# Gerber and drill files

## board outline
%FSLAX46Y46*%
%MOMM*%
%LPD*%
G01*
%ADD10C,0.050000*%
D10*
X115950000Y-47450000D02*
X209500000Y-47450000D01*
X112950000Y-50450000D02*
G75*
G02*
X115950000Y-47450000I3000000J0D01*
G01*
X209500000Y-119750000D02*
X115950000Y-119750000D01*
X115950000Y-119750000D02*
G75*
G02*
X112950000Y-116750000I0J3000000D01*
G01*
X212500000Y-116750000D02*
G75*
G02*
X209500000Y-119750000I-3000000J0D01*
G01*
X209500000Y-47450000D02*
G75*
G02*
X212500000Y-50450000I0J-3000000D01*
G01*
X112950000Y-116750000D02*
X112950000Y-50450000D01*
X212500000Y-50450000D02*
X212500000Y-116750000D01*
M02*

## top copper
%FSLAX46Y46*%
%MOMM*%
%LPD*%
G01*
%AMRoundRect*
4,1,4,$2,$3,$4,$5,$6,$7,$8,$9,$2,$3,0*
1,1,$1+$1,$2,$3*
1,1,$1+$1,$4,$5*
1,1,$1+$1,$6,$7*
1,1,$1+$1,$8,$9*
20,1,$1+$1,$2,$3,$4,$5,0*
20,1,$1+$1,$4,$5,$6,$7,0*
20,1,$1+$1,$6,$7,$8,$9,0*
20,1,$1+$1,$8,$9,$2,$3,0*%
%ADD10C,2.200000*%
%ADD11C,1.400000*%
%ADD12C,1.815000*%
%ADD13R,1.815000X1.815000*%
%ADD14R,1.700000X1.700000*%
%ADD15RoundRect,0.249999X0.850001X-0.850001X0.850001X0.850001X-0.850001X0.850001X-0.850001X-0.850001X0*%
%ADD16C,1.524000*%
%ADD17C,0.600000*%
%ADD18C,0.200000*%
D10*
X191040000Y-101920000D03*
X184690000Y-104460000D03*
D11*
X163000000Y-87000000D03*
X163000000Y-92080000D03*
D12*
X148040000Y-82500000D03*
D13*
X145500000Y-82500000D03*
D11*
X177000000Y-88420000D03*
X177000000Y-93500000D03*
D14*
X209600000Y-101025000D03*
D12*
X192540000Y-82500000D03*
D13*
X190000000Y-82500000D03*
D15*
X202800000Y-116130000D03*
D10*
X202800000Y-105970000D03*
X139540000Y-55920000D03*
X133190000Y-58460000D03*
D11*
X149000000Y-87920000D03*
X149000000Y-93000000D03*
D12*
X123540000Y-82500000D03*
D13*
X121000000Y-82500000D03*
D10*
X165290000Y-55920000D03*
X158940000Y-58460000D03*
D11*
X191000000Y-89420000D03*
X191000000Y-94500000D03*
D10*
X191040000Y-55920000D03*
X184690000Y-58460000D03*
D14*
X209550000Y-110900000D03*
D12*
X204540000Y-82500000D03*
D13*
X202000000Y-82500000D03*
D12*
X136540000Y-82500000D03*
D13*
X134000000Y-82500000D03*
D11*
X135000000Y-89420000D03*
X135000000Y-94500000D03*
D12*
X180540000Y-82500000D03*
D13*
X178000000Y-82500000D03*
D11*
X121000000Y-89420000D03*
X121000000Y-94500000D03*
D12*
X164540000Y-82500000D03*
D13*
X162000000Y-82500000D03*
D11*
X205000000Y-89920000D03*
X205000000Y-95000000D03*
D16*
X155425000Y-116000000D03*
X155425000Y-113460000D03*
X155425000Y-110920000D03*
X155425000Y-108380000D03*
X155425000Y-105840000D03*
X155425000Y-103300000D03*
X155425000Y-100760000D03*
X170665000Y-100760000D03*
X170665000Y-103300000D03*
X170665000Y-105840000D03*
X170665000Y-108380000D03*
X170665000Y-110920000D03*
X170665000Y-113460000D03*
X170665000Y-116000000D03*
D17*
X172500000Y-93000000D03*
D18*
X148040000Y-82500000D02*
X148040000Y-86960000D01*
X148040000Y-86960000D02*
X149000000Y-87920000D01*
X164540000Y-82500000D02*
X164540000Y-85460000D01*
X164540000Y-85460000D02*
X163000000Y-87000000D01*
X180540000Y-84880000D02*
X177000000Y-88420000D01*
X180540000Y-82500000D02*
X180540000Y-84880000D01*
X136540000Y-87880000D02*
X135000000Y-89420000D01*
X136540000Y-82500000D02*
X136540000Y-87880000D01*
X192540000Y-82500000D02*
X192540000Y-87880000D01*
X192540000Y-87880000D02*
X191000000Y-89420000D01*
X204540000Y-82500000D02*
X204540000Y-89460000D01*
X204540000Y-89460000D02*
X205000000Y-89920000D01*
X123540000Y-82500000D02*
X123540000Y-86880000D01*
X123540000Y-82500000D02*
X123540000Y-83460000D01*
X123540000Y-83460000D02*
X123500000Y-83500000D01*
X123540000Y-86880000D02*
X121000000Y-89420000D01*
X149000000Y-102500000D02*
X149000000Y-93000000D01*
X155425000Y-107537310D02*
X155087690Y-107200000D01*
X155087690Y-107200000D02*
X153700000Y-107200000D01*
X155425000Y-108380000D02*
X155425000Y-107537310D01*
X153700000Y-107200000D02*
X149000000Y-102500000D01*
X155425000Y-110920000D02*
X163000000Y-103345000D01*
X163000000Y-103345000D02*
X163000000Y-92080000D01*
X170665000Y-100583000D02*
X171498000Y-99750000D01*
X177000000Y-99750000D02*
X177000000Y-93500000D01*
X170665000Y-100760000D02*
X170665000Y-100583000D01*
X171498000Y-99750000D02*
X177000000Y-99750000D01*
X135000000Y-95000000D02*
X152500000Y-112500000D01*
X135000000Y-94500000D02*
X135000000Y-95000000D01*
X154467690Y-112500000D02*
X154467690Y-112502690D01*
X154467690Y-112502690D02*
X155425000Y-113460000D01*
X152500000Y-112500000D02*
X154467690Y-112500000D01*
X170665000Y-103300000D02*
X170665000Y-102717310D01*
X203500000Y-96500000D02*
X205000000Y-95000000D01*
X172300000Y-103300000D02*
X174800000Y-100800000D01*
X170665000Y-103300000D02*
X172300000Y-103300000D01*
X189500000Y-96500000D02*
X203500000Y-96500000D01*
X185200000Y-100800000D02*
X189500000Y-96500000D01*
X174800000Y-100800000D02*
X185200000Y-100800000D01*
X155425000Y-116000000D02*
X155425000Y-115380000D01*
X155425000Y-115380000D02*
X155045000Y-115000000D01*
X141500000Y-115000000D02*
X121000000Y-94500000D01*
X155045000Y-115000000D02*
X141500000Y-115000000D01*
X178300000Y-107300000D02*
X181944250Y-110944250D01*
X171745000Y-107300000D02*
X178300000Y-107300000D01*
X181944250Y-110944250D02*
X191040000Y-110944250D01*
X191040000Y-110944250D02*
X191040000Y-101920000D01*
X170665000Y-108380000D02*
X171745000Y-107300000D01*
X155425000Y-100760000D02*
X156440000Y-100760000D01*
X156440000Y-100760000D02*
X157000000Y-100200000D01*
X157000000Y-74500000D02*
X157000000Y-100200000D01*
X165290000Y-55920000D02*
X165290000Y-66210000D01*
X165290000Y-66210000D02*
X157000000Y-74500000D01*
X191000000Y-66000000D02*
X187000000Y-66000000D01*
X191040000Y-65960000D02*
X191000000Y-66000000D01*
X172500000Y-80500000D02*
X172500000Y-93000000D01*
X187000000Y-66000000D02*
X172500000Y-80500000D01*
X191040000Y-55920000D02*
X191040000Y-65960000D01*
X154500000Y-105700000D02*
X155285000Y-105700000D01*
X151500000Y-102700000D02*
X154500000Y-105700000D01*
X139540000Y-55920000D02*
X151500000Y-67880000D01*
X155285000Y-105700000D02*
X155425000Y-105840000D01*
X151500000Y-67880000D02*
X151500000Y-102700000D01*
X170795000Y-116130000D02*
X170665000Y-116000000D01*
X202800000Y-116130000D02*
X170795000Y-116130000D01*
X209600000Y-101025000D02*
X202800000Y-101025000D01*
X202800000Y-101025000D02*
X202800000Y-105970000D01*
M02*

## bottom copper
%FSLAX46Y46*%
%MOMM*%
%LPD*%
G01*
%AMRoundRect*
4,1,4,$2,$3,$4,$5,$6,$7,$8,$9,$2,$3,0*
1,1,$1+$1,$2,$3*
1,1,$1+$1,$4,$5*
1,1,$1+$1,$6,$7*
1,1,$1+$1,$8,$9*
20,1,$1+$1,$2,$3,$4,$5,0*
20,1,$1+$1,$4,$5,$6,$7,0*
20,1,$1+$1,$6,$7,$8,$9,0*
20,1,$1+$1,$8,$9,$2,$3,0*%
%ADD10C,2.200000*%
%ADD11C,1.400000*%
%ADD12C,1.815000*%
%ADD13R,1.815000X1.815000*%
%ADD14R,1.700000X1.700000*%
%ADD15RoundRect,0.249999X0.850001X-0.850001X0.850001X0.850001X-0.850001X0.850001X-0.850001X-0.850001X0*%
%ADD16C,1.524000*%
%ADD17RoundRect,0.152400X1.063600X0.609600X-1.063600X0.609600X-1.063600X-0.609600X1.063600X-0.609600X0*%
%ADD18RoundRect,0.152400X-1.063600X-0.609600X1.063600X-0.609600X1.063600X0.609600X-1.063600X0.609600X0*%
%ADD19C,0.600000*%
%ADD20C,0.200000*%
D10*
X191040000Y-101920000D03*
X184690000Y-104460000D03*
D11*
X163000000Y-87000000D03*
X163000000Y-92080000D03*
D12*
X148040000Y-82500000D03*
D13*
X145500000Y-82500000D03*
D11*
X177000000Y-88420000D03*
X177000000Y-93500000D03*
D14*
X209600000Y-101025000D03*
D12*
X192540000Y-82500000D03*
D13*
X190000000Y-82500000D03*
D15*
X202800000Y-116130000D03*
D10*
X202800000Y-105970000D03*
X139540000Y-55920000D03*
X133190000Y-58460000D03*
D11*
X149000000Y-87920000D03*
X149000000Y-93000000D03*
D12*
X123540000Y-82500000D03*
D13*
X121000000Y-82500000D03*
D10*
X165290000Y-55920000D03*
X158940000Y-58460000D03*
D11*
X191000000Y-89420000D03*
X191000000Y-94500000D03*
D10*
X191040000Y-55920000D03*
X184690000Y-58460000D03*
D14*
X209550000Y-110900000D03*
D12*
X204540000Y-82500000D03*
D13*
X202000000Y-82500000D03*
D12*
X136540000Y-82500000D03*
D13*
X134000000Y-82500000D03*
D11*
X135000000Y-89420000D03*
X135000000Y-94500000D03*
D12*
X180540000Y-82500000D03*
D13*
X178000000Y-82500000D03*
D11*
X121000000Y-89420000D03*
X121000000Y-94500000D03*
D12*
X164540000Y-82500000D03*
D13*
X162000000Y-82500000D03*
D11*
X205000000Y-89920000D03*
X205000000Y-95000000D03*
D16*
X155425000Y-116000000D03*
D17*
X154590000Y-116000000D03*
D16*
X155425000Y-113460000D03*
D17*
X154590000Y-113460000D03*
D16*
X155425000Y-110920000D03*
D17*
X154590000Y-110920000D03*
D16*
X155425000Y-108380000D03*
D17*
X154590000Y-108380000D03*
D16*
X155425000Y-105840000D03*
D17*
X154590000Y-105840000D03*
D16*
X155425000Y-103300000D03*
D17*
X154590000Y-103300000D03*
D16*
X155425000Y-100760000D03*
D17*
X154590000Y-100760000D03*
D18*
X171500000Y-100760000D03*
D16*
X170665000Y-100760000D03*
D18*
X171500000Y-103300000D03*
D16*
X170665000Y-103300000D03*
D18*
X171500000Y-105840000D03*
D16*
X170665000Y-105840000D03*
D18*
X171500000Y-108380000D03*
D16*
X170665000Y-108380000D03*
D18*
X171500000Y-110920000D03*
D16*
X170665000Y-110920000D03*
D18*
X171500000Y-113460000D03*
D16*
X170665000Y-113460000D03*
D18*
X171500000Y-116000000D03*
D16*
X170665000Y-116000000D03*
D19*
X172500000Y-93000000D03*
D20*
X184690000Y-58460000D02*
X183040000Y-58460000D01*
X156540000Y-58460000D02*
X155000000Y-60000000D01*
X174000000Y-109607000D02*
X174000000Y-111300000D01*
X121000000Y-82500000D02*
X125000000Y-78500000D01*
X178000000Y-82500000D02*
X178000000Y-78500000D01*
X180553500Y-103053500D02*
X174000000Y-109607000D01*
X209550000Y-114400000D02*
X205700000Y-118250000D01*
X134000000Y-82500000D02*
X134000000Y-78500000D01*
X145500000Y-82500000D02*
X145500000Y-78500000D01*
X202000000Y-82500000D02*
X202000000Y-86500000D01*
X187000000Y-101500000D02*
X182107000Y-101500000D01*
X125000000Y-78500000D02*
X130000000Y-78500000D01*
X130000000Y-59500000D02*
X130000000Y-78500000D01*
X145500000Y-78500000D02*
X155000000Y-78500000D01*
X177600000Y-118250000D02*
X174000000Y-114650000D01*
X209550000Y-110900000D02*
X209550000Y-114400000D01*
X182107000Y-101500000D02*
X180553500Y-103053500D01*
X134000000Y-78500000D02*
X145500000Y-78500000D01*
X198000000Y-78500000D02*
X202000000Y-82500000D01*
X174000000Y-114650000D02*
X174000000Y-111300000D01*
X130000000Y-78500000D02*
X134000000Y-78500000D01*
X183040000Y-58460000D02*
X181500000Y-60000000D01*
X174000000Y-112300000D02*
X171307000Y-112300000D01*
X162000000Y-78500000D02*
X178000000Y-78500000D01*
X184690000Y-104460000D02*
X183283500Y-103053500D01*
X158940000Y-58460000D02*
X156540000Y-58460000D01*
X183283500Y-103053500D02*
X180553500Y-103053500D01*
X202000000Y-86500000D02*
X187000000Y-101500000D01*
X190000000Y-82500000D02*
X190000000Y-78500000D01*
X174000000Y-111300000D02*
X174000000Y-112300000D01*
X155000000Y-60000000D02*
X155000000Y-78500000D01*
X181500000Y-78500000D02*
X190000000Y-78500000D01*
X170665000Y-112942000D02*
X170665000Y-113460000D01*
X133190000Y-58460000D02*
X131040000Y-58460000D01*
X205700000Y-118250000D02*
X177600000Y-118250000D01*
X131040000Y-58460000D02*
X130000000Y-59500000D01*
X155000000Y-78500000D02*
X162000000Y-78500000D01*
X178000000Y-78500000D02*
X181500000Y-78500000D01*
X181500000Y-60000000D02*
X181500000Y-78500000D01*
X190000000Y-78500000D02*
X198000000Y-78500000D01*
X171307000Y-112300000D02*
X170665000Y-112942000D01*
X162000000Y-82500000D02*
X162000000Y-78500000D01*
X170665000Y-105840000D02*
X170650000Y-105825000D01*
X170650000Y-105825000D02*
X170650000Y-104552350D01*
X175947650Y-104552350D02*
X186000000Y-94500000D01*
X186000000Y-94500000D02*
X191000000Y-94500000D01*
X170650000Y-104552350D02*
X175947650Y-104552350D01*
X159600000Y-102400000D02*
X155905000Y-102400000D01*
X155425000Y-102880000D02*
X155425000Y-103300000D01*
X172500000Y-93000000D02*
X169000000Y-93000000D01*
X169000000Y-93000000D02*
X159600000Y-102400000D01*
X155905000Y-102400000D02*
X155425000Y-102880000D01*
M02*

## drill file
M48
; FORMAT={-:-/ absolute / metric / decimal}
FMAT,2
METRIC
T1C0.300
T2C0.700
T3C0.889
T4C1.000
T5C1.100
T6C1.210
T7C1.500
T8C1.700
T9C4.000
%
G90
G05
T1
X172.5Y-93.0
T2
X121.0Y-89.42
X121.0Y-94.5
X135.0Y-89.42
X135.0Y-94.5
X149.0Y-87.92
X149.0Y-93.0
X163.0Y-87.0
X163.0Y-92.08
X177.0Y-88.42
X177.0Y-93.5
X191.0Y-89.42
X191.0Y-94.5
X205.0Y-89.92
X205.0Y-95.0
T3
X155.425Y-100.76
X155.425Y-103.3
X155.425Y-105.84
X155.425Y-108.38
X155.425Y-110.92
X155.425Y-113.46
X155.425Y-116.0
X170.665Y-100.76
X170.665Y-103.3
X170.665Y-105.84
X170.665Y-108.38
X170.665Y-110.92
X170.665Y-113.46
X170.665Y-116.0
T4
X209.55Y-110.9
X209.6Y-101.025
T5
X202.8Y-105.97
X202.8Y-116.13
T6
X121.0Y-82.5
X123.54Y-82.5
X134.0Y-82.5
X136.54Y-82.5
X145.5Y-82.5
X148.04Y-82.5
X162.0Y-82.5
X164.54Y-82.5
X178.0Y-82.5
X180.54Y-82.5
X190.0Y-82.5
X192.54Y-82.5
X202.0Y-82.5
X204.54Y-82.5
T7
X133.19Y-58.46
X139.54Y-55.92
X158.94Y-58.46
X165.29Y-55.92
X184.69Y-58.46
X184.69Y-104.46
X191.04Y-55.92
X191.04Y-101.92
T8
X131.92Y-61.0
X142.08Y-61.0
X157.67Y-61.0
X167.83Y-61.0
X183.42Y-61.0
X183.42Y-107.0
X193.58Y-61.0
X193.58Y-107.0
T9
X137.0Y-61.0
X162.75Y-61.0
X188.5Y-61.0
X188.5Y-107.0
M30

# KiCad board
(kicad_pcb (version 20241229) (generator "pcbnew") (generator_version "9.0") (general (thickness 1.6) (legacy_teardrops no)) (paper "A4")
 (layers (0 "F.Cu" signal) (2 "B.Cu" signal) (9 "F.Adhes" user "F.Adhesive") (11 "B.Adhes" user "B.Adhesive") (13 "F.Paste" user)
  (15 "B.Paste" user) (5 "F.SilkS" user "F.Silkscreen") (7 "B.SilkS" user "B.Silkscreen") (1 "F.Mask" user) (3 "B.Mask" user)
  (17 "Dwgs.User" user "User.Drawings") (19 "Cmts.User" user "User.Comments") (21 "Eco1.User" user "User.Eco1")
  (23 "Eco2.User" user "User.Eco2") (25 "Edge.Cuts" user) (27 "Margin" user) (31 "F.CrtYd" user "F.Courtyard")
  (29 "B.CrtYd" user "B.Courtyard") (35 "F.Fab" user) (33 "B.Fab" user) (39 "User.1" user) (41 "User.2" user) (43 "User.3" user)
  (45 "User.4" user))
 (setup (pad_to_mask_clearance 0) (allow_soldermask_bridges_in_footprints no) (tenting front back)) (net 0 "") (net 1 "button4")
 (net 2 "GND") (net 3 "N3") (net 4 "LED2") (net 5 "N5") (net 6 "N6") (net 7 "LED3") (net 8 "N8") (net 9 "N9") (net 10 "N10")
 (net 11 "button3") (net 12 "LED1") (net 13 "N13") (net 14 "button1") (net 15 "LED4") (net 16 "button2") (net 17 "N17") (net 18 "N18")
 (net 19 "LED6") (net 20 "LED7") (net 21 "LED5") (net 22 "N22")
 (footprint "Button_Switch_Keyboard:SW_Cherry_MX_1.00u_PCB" (layer "F.Cu") (at 191.04 101.92)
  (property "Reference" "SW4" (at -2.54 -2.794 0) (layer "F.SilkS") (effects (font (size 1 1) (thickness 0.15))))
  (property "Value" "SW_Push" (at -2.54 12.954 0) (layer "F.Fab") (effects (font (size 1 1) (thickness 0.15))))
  (pad "" np_thru_hole circle (at -7.62 5.08) (size 1.7 1.7) (drill 1.7) (layers "*.Cu" "*.Mask"))
  (pad "" np_thru_hole circle (at -2.54 5.08) (size 4 4) (drill 4) (layers "*.Cu" "*.Mask"))
  (pad "" np_thru_hole circle (at 2.54 5.08) (size 1.7 1.7) (drill 1.7) (layers "*.Cu" "*.Mask"))
  (pad "1" thru_hole circle (at 0 0) (size 2.2 2.2) (drill 1.5) (layers "*.Cu" "*.Mask") (remove_unused_layers no) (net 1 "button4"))
  (pad "2" thru_hole circle (at -6.35 2.54) (size 2.2 2.2) (drill 1.5) (layers "*.Cu" "*.Mask") (remove_unused_layers no) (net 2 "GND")))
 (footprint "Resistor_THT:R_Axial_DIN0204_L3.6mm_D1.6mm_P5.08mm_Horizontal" (layer "F.Cu") (at 163 87 -90)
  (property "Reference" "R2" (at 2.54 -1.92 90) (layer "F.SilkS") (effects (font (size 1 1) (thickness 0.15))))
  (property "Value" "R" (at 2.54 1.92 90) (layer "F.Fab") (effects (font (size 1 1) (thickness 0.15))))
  (pad "1" thru_hole circle (at 0 0 270) (size 1.4 1.4) (drill 0.7) (layers "*.Cu" "*.Mask") (remove_unused_layers no) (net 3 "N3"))
  (pad "2" thru_hole circle (at 5.08 0 270) (size 1.4 1.4) (drill 0.7) (layers "*.Cu" "*.Mask") (remove_unused_layers no) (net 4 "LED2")))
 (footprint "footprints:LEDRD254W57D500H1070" (layer "F.Cu") (at 146.77 82.5)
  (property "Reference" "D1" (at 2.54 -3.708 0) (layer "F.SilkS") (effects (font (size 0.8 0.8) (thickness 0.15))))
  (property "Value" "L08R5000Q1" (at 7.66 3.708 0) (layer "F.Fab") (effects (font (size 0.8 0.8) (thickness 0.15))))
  (pad "A" thru_hole circle (at 1.27 0) (size 1.815 1.815) (drill 1.21) (layers "*.Cu" "*.Mask") (remove_unused_layers no) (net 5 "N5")
   (solder_mask_margin 0.102))
  (pad "C" thru_hole rect (at -1.27 0) (size 1.815 1.815) (drill 1.21) (layers "*.Cu" "*.Mask") (remove_unused_layers no) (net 2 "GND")
   (solder_mask_margin 0.102)))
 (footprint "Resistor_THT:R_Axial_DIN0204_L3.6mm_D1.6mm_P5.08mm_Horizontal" (layer "F.Cu") (at 177 88.42 -90)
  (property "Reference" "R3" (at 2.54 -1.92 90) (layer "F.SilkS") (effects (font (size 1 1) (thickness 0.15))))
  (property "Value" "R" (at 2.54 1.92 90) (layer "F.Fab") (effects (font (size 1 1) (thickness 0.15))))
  (pad "1" thru_hole circle (at 0 0 270) (size 1.4 1.4) (drill 0.7) (layers "*.Cu" "*.Mask") (remove_unused_layers no) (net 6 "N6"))
  (pad "2" thru_hole circle (at 5.08 0 270) (size 1.4 1.4) (drill 0.7) (layers "*.Cu" "*.Mask") (remove_unused_layers no) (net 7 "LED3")))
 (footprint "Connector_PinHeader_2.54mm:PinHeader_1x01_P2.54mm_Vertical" (layer "F.Cu") (at 209.6 101.025)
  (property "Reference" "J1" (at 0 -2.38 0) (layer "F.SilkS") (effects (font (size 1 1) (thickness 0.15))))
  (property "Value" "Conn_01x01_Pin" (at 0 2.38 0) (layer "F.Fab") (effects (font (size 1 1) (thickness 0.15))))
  (pad "1" thru_hole rect (at 0 0) (size 1.7 1.7) (drill 1) (layers "*.Cu" "*.Mask") (remove_unused_layers no) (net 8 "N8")))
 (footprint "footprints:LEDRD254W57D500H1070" (layer "F.Cu") (at 191.27 82.5)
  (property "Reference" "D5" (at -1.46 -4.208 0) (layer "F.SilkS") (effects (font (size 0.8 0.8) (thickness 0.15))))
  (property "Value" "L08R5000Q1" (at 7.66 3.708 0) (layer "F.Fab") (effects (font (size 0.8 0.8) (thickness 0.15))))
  (pad "A" thru_hole circle (at 1.27 0) (size 1.815 1.815) (drill 1.21) (layers "*.Cu" "*.Mask") (remove_unused_layers no) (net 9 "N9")
   (solder_mask_margin 0.102))
  (pad "C" thru_hole rect (at -1.27 0) (size 1.815 1.815) (drill 1.21) (layers "*.Cu" "*.Mask") (remove_unused_layers no) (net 2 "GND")
   (solder_mask_margin 0.102)))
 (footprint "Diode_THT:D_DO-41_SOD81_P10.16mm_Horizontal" (layer "F.Cu") (at 202.8 116.13 90)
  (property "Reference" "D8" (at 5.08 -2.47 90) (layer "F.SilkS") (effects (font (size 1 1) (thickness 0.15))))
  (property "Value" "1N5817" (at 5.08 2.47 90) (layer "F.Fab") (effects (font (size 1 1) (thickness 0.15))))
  (pad "1" thru_hole roundrect (at 0 0 90) (size 2.2 2.2) (drill 1.1) (layers "*.Cu" "*.Mask") (remove_unused_layers no)
   (roundrect_rratio 0.113636) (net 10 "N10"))
  (pad "2" thru_hole circle (at 10.16 0 90) (size 2.2 2.2) (drill 1.1) (layers "*.Cu" "*.Mask") (remove_unused_layers no) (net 8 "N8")))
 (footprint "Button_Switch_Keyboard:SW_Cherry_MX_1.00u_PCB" (layer "F.Cu") (at 139.54 55.92)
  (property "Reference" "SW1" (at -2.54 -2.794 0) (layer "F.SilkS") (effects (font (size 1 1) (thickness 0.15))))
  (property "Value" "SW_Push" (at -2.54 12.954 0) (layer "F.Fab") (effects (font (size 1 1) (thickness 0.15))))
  (pad "" np_thru_hole circle (at -7.62 5.08) (size 1.7 1.7) (drill 1.7) (layers "*.Cu" "*.Mask"))
  (pad "" np_thru_hole circle (at -2.54 5.08) (size 4 4) (drill 4) (layers "*.Cu" "*.Mask"))
  (pad "" np_thru_hole circle (at 2.54 5.08) (size 1.7 1.7) (drill 1.7) (layers "*.Cu" "*.Mask"))
  (pad "1" thru_hole circle (at 0 0) (size 2.2 2.2) (drill 1.5) (layers "*.Cu" "*.Mask") (remove_unused_layers no) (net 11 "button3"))
  (pad "2" thru_hole circle (at -6.35 2.54) (size 2.2 2.2) (drill 1.5) (layers "*.Cu" "*.Mask") (remove_unused_layers no) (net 2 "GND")))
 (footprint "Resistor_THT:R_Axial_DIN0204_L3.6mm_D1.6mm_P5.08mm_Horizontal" (layer "F.Cu") (at 149 87.92 -90)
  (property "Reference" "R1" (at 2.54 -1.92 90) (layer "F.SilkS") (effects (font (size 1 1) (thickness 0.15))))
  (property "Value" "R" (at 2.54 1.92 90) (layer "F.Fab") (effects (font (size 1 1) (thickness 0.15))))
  (pad "1" thru_hole circle (at 0 0 270) (size 1.4 1.4) (drill 0.7) (layers "*.Cu" "*.Mask") (remove_unused_layers no) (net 5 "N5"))
  (pad "2" thru_hole circle (at 5.08 0 270) (size 1.4 1.4) (drill 0.7) (layers "*.Cu" "*.Mask") (remove_unused_layers no) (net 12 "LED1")))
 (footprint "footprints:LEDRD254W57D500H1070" (layer "F.Cu") (at 122.27 82.5)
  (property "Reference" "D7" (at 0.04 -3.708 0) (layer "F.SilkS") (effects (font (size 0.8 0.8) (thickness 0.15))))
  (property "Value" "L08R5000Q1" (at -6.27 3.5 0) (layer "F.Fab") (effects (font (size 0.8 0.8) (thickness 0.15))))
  (pad "A" thru_hole circle (at 1.27 0) (size 1.815 1.815) (drill 1.21) (layers "*.Cu" "*.Mask") (remove_unused_layers no) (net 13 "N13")
   (solder_mask_margin 0.102))
  (pad "C" thru_hole rect (at -1.27 0) (size 1.815 1.815) (drill 1.21) (layers "*.Cu" "*.Mask") (remove_unused_layers no) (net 2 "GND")
   (solder_mask_margin 0.102)))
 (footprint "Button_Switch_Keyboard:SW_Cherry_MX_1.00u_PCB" (layer "F.Cu") (at 165.29 55.92)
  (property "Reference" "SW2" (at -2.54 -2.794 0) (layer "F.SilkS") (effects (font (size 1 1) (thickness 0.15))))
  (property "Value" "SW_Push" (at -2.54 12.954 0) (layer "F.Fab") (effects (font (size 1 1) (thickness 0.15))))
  (pad "" np_thru_hole circle (at -7.62 5.08) (size 1.7 1.7) (drill 1.7) (layers "*.Cu" "*.Mask"))
  (pad "" np_thru_hole circle (at -2.54 5.08) (size 4 4) (drill 4) (layers "*.Cu" "*.Mask"))
  (pad "" np_thru_hole circle (at 2.54 5.08) (size 1.7 1.7) (drill 1.7) (layers "*.Cu" "*.Mask"))
  (pad "1" thru_hole circle (at 0 0) (size 2.2 2.2) (drill 1.5) (layers "*.Cu" "*.Mask") (remove_unused_layers no) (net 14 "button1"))
  (pad "2" thru_hole circle (at -6.35 2.54) (size 2.2 2.2) (drill 1.5) (layers "*.Cu" "*.Mask") (remove_unused_layers no) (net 2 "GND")))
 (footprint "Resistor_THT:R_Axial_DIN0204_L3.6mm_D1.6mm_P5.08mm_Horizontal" (layer "F.Cu") (at 191 89.42 -90)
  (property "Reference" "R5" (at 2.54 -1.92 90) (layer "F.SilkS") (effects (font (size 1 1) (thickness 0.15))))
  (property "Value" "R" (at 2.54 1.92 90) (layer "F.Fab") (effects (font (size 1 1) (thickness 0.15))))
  (pad "1" thru_hole circle (at 0 0 270) (size 1.4 1.4) (drill 0.7) (layers "*.Cu" "*.Mask") (remove_unused_layers no) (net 9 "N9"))
  (pad "2" thru_hole circle (at 5.08 0 270) (size 1.4 1.4) (drill 0.7) (layers "*.Cu" "*.Mask") (remove_unused_layers no) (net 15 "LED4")))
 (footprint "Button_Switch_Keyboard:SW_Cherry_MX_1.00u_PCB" (layer "F.Cu") (at 191.04 55.92)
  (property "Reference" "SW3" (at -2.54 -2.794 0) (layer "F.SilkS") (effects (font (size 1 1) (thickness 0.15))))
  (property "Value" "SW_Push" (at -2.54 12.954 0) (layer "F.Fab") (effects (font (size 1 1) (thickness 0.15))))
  (pad "" np_thru_hole circle (at -7.62 5.08) (size 1.7 1.7) (drill 1.7) (layers "*.Cu" "*.Mask"))
  (pad "" np_thru_hole circle (at -2.54 5.08) (size 4 4) (drill 4) (layers "*.Cu" "*.Mask"))
  (pad "" np_thru_hole circle (at 2.54 5.08) (size 1.7 1.7) (drill 1.7) (layers "*.Cu" "*.Mask"))
  (pad "1" thru_hole circle (at 0 0) (size 2.2 2.2) (drill 1.5) (layers "*.Cu" "*.Mask") (remove_unused_layers no) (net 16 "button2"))
  (pad "2" thru_hole circle (at -6.35 2.54) (size 2.2 2.2) (drill 1.5) (layers "*.Cu" "*.Mask") (remove_unused_layers no) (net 2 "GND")))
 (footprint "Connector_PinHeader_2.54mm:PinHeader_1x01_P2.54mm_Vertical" (layer "F.Cu") (at 209.55 110.9)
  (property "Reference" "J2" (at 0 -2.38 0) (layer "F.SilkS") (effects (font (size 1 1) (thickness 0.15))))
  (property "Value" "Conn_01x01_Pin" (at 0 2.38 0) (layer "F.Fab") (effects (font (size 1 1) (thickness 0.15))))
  (pad "1" thru_hole rect (at 0 0) (size 1.7 1.7) (drill 1) (layers "*.Cu" "*.Mask") (remove_unused_layers no) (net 2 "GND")))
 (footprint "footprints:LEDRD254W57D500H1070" (layer "F.Cu") (at 203.27 82.5)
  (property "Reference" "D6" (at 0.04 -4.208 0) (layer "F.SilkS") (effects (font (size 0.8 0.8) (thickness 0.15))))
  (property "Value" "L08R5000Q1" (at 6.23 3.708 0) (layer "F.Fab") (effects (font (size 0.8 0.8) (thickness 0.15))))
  (pad "A" thru_hole circle (at 1.27 0) (size 1.815 1.815) (drill 1.21) (layers "*.Cu" "*.Mask") (remove_unused_layers no) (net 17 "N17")
   (solder_mask_margin 0.102))
  (pad "C" thru_hole rect (at -1.27 0) (size 1.815 1.815) (drill 1.21) (layers "*.Cu" "*.Mask") (remove_unused_layers no) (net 2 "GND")
   (solder_mask_margin 0.102)))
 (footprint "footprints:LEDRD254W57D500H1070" (layer "F.Cu") (at 135.27 82.5)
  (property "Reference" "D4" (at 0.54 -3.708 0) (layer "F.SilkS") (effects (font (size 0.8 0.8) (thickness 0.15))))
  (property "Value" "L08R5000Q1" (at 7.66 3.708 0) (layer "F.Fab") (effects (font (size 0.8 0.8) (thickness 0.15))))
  (pad "A" thru_hole circle (at 1.27 0) (size 1.815 1.815) (drill 1.21) (layers "*.Cu" "*.Mask") (remove_unused_layers no) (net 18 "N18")
   (solder_mask_margin 0.102))
  (pad "C" thru_hole rect (at -1.27 0) (size 1.815 1.815) (drill 1.21) (layers "*.Cu" "*.Mask") (remove_unused_layers no) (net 2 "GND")
   (solder_mask_margin 0.102)))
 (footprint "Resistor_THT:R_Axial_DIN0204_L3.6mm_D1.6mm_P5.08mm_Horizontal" (layer "F.Cu") (at 135 89.42 -90)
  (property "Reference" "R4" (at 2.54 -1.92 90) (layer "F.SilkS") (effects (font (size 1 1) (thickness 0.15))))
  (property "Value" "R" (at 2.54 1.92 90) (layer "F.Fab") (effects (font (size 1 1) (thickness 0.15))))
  (pad "1" thru_hole circle (at 0 0 270) (size 1.4 1.4) (drill 0.7) (layers "*.Cu" "*.Mask") (remove_unused_layers no) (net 18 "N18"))
  (pad "2" thru_hole circle (at 5.08 0 270) (size 1.4 1.4) (drill 0.7) (layers "*.Cu" "*.Mask") (remove_unused_layers no) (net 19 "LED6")))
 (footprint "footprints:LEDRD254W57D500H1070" (layer "F.Cu") (at 179.27 82.5)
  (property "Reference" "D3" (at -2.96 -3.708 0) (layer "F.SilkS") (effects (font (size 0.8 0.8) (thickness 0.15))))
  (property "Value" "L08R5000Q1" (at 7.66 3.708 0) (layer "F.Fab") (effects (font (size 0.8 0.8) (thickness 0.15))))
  (pad "A" thru_hole circle (at 1.27 0) (size 1.815 1.815) (drill 1.21) (layers "*.Cu" "*.Mask") (remove_unused_layers no) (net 6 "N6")
   (solder_mask_margin 0.102))
  (pad "C" thru_hole rect (at -1.27 0) (size 1.815 1.815) (drill 1.21) (layers "*.Cu" "*.Mask") (remove_unused_layers no) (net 2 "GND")
   (solder_mask_margin 0.102)))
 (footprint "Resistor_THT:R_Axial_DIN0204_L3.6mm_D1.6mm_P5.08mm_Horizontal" (layer "F.Cu") (at 121 89.42 -90)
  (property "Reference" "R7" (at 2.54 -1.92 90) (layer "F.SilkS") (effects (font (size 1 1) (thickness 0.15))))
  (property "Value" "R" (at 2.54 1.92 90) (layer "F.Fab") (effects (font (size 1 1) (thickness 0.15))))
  (pad "1" thru_hole circle (at 0 0 270) (size 1.4 1.4) (drill 0.7) (layers "*.Cu" "*.Mask") (remove_unused_layers no) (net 13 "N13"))
  (pad "2" thru_hole circle (at 5.08 0 270) (size 1.4 1.4) (drill 0.7) (layers "*.Cu" "*.Mask") (remove_unused_layers no) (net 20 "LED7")))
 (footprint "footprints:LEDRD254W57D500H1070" (layer "F.Cu") (at 163.27 82.5)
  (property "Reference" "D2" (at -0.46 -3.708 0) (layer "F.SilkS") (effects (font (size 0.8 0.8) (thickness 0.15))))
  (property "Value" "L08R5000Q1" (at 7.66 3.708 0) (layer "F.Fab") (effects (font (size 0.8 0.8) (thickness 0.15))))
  (pad "A" thru_hole circle (at 1.27 0) (size 1.815 1.815) (drill 1.21) (layers "*.Cu" "*.Mask") (remove_unused_layers no) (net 3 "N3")
   (solder_mask_margin 0.102))
  (pad "C" thru_hole rect (at -1.27 0) (size 1.815 1.815) (drill 1.21) (layers "*.Cu" "*.Mask") (remove_unused_layers no) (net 2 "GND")
   (solder_mask_margin 0.102)))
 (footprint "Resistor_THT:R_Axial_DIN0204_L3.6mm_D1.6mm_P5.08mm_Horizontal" (layer "F.Cu") (at 205 89.92 -90)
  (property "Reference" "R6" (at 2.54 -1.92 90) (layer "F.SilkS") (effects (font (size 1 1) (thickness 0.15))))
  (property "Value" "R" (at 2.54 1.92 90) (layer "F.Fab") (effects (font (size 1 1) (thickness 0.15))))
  (pad "1" thru_hole circle (at 0 0 270) (size 1.4 1.4) (drill 0.7) (layers "*.Cu" "*.Mask") (remove_unused_layers no) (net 17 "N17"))
  (pad "2" thru_hole circle (at 5.08 0 270) (size 1.4 1.4) (drill 0.7) (layers "*.Cu" "*.Mask") (remove_unused_layers no) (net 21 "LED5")))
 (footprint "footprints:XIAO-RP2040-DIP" (layer "B.Cu") (at 163.045 108.38 -90)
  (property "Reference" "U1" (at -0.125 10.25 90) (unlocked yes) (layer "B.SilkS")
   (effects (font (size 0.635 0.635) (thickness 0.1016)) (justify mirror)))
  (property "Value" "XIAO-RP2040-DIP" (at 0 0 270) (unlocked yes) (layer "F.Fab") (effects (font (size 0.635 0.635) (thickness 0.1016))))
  (pad "1" thru_hole circle (at 7.62 7.62 180) (size 1.524 1.524) (drill 0.889) (layers "*.Cu" "*.Mask") (remove_unused_layers no)
   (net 20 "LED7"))
  (pad "1" smd roundrect (at 7.62 8.455 180) (size 2.432 1.524) (layers "B.Cu" "B.Mask") (roundrect_rratio 0.1) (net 20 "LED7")
   (thermal_bridge_angle 45))
  (pad "2" thru_hole circle (at 5.08 7.62 180) (size 1.524 1.524) (drill 0.889) (layers "*.Cu" "*.Mask") (remove_unused_layers no)
   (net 19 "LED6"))
  (pad "2" smd roundrect (at 5.08 8.455 180) (size 2.432 1.524) (layers "B.Cu" "B.Mask") (roundrect_rratio 0.1) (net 19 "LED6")
   (thermal_bridge_angle 45))
  (pad "3" thru_hole circle (at 2.54 7.62 180) (size 1.524 1.524) (drill 0.889) (layers "*.Cu" "*.Mask") (remove_unused_layers no)
   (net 4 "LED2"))
  (pad "3" smd roundrect (at 2.54 8.455 180) (size 2.432 1.524) (layers "B.Cu" "B.Mask") (roundrect_rratio 0.1) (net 4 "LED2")
   (thermal_bridge_angle 45))
  (pad "4" thru_hole circle (at 0 7.62 180) (size 1.524 1.524) (drill 0.889) (layers "*.Cu" "*.Mask") (remove_unused_layers no)
   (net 12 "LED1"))
  (pad "4" smd roundrect (at 0 8.455 180) (size 2.432 1.524) (layers "B.Cu" "B.Mask") (roundrect_rratio 0.1) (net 12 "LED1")
   (thermal_bridge_angle 45))
  (pad "5" thru_hole circle (at -2.54 7.62 180) (size 1.524 1.524) (drill 0.889) (layers "*.Cu" "*.Mask") (remove_unused_layers no)
   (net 11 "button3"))
  (pad "5" smd roundrect (at -2.54 8.455 180) (size 2.432 1.524) (layers "B.Cu" "B.Mask") (roundrect_rratio 0.1) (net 11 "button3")
   (thermal_bridge_angle 45))
  (pad "6" thru_hole circle (at -5.08 7.62 180) (size 1.524 1.524) (drill 0.889) (layers "*.Cu" "*.Mask") (remove_unused_layers no)
   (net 16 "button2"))
  (pad "6" smd roundrect (at -5.08 8.455 180) (size 2.432 1.524) (layers "B.Cu" "B.Mask") (roundrect_rratio 0.1) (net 16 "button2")
   (thermal_bridge_angle 45))
  (pad "7" thru_hole circle (at -7.62 7.62 180) (size 1.524 1.524) (drill 0.889) (layers "*.Cu" "*.Mask") (remove_unused_layers no)
   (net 14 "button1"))
  (pad "7" smd roundrect (at -7.62 8.455 180) (size 2.432 1.524) (layers "B.Cu" "B.Mask") (roundrect_rratio 0.1) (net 14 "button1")
   (thermal_bridge_angle 45))
  (pad "8" smd roundrect (at -7.62 -8.455) (size 2.432 1.524) (layers "B.Cu" "B.Mask") (roundrect_rratio 0.1) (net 7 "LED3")
   (thermal_bridge_angle 45))
  (pad "8" thru_hole circle (at -7.62 -7.62) (size 1.524 1.524) (drill 0.889) (layers "*.Cu" "*.Mask") (remove_unused_layers no)
   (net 7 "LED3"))
  (pad "9" smd roundrect (at -5.08 -8.455) (size 2.432 1.524) (layers "B.Cu" "B.Mask") (roundrect_rratio 0.1) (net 21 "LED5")
   (thermal_bridge_angle 45))
  (pad "9" thru_hole circle (at -5.08 -7.62) (size 1.524 1.524) (drill 0.889) (layers "*.Cu" "*.Mask") (remove_unused_layers no)
   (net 21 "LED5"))
  (pad "10" smd roundrect (at -2.54 -8.455) (size 2.432 1.524) (layers "B.Cu" "B.Mask") (roundrect_rratio 0.1) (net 15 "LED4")
   (thermal_bridge_angle 45))
  (pad "10" thru_hole circle (at -2.54 -7.62) (size 1.524 1.524) (drill 0.889) (layers "*.Cu" "*.Mask") (remove_unused_layers no)
   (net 15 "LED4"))
  (pad "11" smd roundrect (at 0 -8.455) (size 2.432 1.524) (layers "B.Cu" "B.Mask") (roundrect_rratio 0.1) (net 1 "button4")
   (thermal_bridge_angle 45))
  (pad "11" thru_hole circle (at 0 -7.62) (size 1.524 1.524) (drill 0.889) (layers "*.Cu" "*.Mask") (remove_unused_layers no)
   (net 1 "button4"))
  (pad "12" smd roundrect (at 2.54 -8.455) (size 2.432 1.524) (layers "B.Cu" "B.Mask") (roundrect_rratio 0.1) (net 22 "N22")
   (thermal_bridge_angle 45))
  (pad "12" thru_hole circle (at 2.54 -7.62) (size 1.524 1.524) (drill 0.889) (layers "*.Cu" "*.Mask") (remove_unused_layers no)
   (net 22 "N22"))
  (pad "13" smd roundrect (at 5.08 -8.455) (size 2.432 1.524) (layers "B.Cu" "B.Mask") (roundrect_rratio 0.1) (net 2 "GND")
   (thermal_bridge_angle 45))
  (pad "13" thru_hole circle (at 5.08 -7.62) (size 1.524 1.524) (drill 0.889) (layers "*.Cu" "*.Mask") (remove_unused_layers no)
   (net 2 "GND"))
  (pad "14" smd roundrect (at 7.62 -8.455) (size 2.432 1.524) (layers "B.Cu" "B.Mask") (roundrect_rratio 0.1) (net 10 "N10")
   (thermal_bridge_angle 45))
  (pad "14" thru_hole circle (at 7.62 -7.62) (size 1.524 1.524) (drill 0.889) (layers "*.Cu" "*.Mask") (remove_unused_layers no)
   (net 10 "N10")))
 (gr_line (start 115.95 47.45) (end 209.5 47.45) (stroke (width 0.05) (type default)) (layer "Edge.Cuts"))
 (gr_arc (start 112.95 50.45) (mid 113.82868 48.32868) (end 115.95 47.45) (stroke (width 0.05) (type default)) (layer "Edge.Cuts"))
 (gr_line (start 209.5 119.75) (end 115.95 119.75) (stroke (width 0.05) (type default)) (layer "Edge.Cuts"))
 (gr_arc (start 115.95 119.75) (mid 113.82868 118.87132) (end 112.95 116.75) (stroke (width 0.05) (type default)) (layer "Edge.Cuts"))
 (gr_arc (start 212.5 116.75) (mid 211.62132 118.87132) (end 209.5 119.75) (stroke (width 0.05) (type default)) (layer "Edge.Cuts"))
 (gr_arc (start 209.5 47.45) (mid 211.62132 48.32868) (end 212.5 50.45) (stroke (width 0.05) (type default)) (layer "Edge.Cuts"))
 (gr_line (start 112.95 116.75) (end 112.95 50.45) (stroke (width 0.05) (type default)) (layer "Edge.Cuts"))
 (gr_line (start 212.5 50.45) (end 212.5 116.75) (stroke (width 0.05) (type default)) (layer "Edge.Cuts"))
 (segment (start 184.69 58.46) (end 183.04 58.46) (width 0.2) (layer "B.Cu") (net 2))
 (segment (start 156.54 58.46) (end 155 60) (width 0.2) (layer "B.Cu") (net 2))
 (segment (start 174 109.607) (end 174 111.3) (width 0.2) (layer "B.Cu") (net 2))
 (segment (start 121 82.5) (end 125 78.5) (width 0.2) (layer "B.Cu") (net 2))
 (segment (start 178 82.5) (end 178 78.5) (width 0.2) (layer "B.Cu") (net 2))
 (segment (start 180.5535 103.0535) (end 174 109.607) (width 0.2) (layer "B.Cu") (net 2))
 (segment (start 209.55 114.4) (end 205.7 118.25) (width 0.2) (layer "B.Cu") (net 2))
 (segment (start 134 82.5) (end 134 78.5) (width 0.2) (layer "B.Cu") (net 2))
 (segment (start 145.5 82.5) (end 145.5 78.5) (width 0.2) (layer "B.Cu") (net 2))
 (segment (start 202 82.5) (end 202 86.5) (width 0.2) (layer "B.Cu") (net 2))
 (segment (start 187 101.5) (end 182.107 101.5) (width 0.2) (layer "B.Cu") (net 2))
 (segment (start 125 78.5) (end 130 78.5) (width 0.2) (layer "B.Cu") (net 2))
 (segment (start 130 59.5) (end 130 78.5) (width 0.2) (layer "B.Cu") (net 2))
 (segment (start 145.5 78.5) (end 155 78.5) (width 0.2) (layer "B.Cu") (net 2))
 (segment (start 177.6 118.25) (end 174 114.65) (width 0.2) (layer "B.Cu") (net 2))
 (segment (start 209.55 110.9) (end 209.55 114.4) (width 0.2) (layer "B.Cu") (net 2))
 (segment (start 182.107 101.5) (end 180.5535 103.0535) (width 0.2) (layer "B.Cu") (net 2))
 (segment (start 134 78.5) (end 145.5 78.5) (width 0.2) (layer "B.Cu") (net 2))
 (segment (start 198 78.5) (end 202 82.5) (width 0.2) (layer "B.Cu") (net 2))
 (segment (start 174 114.65) (end 174 111.3) (width 0.2) (layer "B.Cu") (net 2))
 (segment (start 130 78.5) (end 134 78.5) (width 0.2) (layer "B.Cu") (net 2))
 (segment (start 183.04 58.46) (end 181.5 60) (width 0.2) (layer "B.Cu") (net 2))
 (segment (start 174 112.3) (end 171.307 112.3) (width 0.2) (layer "B.Cu") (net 2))
 (segment (start 162 78.5) (end 178 78.5) (width 0.2) (layer "B.Cu") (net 2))
 (segment (start 184.69 104.46) (end 183.2835 103.0535) (width 0.2) (layer "B.Cu") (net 2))
 (segment (start 158.94 58.46) (end 156.54 58.46) (width 0.2) (layer "B.Cu") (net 2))
 (segment (start 183.2835 103.0535) (end 180.5535 103.0535) (width 0.2) (layer "B.Cu") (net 2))
 (segment (start 202 86.5) (end 187 101.5) (width 0.2) (layer "B.Cu") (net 2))
 (segment (start 190 82.5) (end 190 78.5) (width 0.2) (layer "B.Cu") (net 2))
 (segment (start 174 111.3) (end 174 112.3) (width 0.2) (layer "B.Cu") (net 2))
 (segment (start 155 60) (end 155 78.5) (width 0.2) (layer "B.Cu") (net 2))
 (segment (start 181.5 78.5) (end 190 78.5) (width 0.2) (layer "B.Cu") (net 2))
 (segment (start 170.665 112.942) (end 170.665 113.46) (width 0.2) (layer "B.Cu") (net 2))
 (segment (start 133.19 58.46) (end 131.04 58.46) (width 0.2) (layer "B.Cu") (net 2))
 (segment (start 205.7 118.25) (end 177.6 118.25) (width 0.2) (layer "B.Cu") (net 2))
 (segment (start 131.04 58.46) (end 130 59.5) (width 0.2) (layer "B.Cu") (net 2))
 (segment (start 155 78.5) (end 162 78.5) (width 0.2) (layer "B.Cu") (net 2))
 (segment (start 178 78.5) (end 181.5 78.5) (width 0.2) (layer "B.Cu") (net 2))
 (segment (start 181.5 60) (end 181.5 78.5) (width 0.2) (layer "B.Cu") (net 2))
 (segment (start 190 78.5) (end 198 78.5) (width 0.2) (layer "B.Cu") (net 2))
 (segment (start 171.307 112.3) (end 170.665 112.942) (width 0.2) (layer "B.Cu") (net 2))
 (segment (start 162 82.5) (end 162 78.5) (width 0.2) (layer "B.Cu") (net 2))
 (segment (start 148.04 82.5) (end 148.04 86.96) (width 0.2) (layer "F.Cu") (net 5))
 (segment (start 148.04 86.96) (end 149 87.92) (width 0.2) (layer "F.Cu") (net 5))
 (segment (start 164.54 82.5) (end 164.54 85.46) (width 0.2) (layer "F.Cu") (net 3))
 (segment (start 164.54 85.46) (end 163 87) (width 0.2) (layer "F.Cu") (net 3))
 (segment (start 180.54 84.88) (end 177 88.42) (width 0.2) (layer "F.Cu") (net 6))
 (segment (start 180.54 82.5) (end 180.54 84.88) (width 0.2) (layer "F.Cu") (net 6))
 (segment (start 136.54 87.88) (end 135 89.42) (width 0.2) (layer "F.Cu") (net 18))
 (segment (start 136.54 82.5) (end 136.54 87.88) (width 0.2) (layer "F.Cu") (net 18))
 (segment (start 192.54 82.5) (end 192.54 87.88) (width 0.2) (layer "F.Cu") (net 9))
 (segment (start 192.54 87.88) (end 191 89.42) (width 0.2) (layer "F.Cu") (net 9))
 (segment (start 204.54 82.5) (end 204.54 89.46) (width 0.2) (layer "F.Cu") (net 17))
 (segment (start 204.54 89.46) (end 205 89.92) (width 0.2) (layer "F.Cu") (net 17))
 (segment (start 123.54 82.5) (end 123.54 86.88) (width 0.2) (layer "F.Cu") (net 13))
 (segment (start 123.54 82.5) (end 123.54 83.46) (width 0.2) (layer "F.Cu") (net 13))
 (segment (start 123.54 83.46) (end 123.5 83.5) (width 0.2) (layer "F.Cu") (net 13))
 (segment (start 123.54 86.88) (end 121 89.42) (width 0.2) (layer "F.Cu") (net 13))
 (segment (start 149 102.5) (end 149 93) (width 0.2) (layer "F.Cu") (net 12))
 (segment (start 155.425 107.53731) (end 155.08769 107.2) (width 0.2) (layer "F.Cu") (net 12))
 (segment (start 155.08769 107.2) (end 153.7 107.2) (width 0.2) (layer "F.Cu") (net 12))
 (segment (start 155.425 108.38) (end 155.425 107.53731) (width 0.2) (layer "F.Cu") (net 12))
 (segment (start 153.7 107.2) (end 149 102.5) (width 0.2) (layer "F.Cu") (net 12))
 (segment (start 155.425 110.92) (end 163 103.345) (width 0.2) (layer "F.Cu") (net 4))
 (segment (start 163 103.345) (end 163 92.08) (width 0.2) (layer "F.Cu") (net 4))
 (segment (start 170.665 100.583) (end 171.498 99.75) (width 0.2) (layer "F.Cu") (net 7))
 (segment (start 177 99.75) (end 177 93.5) (width 0.2) (layer "F.Cu") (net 7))
 (segment (start 170.665 100.76) (end 170.665 100.583) (width 0.2) (layer "F.Cu") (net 7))
 (segment (start 171.498 99.75) (end 177 99.75) (width 0.2) (layer "F.Cu") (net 7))
 (segment (start 135 95) (end 152.5 112.5) (width 0.2) (layer "F.Cu") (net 19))
 (segment (start 135 94.5) (end 135 95) (width 0.2) (layer "F.Cu") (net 19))
 (segment (start 154.46769 112.5) (end 154.46769 112.50269) (width 0.2) (layer "F.Cu") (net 19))
 (segment (start 154.46769 112.50269) (end 155.425 113.46) (width 0.2) (layer "F.Cu") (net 19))
 (segment (start 152.5 112.5) (end 154.46769 112.5) (width 0.2) (layer "F.Cu") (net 19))
 (segment (start 170.665 105.84) (end 170.65 105.825) (width 0.2) (layer "B.Cu") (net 15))
 (segment (start 170.65 105.825) (end 170.65 104.55235) (width 0.2) (layer "B.Cu") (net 15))
 (segment (start 175.94765 104.55235) (end 186 94.5) (width 0.2) (layer "B.Cu") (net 15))
 (segment (start 186 94.5) (end 191 94.5) (width 0.2) (layer "B.Cu") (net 15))
 (segment (start 170.65 104.55235) (end 175.94765 104.55235) (width 0.2) (layer "B.Cu") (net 15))
 (segment (start 170.665 103.3) (end 170.665 102.71731) (width 0.2) (layer "F.Cu") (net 21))
 (segment (start 203.5 96.5) (end 205 95) (width 0.2) (layer "F.Cu") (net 21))
 (segment (start 172.3 103.3) (end 174.8 100.8) (width 0.2) (layer "F.Cu") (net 21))
 (segment (start 170.665 103.3) (end 172.3 103.3) (width 0.2) (layer "F.Cu") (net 21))
 (segment (start 189.5 96.5) (end 203.5 96.5) (width 0.2) (layer "F.Cu") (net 21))
 (segment (start 185.2 100.8) (end 189.5 96.5) (width 0.2) (layer "F.Cu") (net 21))
 (segment (start 174.8 100.8) (end 185.2 100.8) (width 0.2) (layer "F.Cu") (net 21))
 (segment (start 155.425 116) (end 155.425 115.38) (width 0.2) (layer "F.Cu") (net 20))
 (segment (start 155.425 115.38) (end 155.045 115) (width 0.2) (layer "F.Cu") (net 20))
 (segment (start 141.5 115) (end 121 94.5) (width 0.2) (layer "F.Cu") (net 20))
 (segment (start 155.045 115) (end 141.5 115) (width 0.2) (layer "F.Cu") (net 20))
 (segment (start 178.3 107.3) (end 181.94425 110.94425) (width 0.2) (layer "F.Cu") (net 1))
 (segment (start 171.745 107.3) (end 178.3 107.3) (width 0.2) (layer "F.Cu") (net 1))
 (segment (start 181.94425 110.94425) (end 191.04 110.94425) (width 0.2) (layer "F.Cu") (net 1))
 (segment (start 191.04 110.94425) (end 191.04 101.92) (width 0.2) (layer "F.Cu") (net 1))
 (segment (start 170.665 108.38) (end 171.745 107.3) (width 0.2) (layer "F.Cu") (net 1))
 (segment (start 155.425 100.76) (end 156.44 100.76) (width 0.2) (layer "F.Cu") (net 14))
 (segment (start 156.44 100.76) (end 157 100.2) (width 0.2) (layer "F.Cu") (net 14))
 (segment (start 157 74.5) (end 157 100.2) (width 0.2) (layer "F.Cu") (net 14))
 (segment (start 165.29 55.92) (end 165.29 66.21) (width 0.2) (layer "F.Cu") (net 14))
 (segment (start 165.29 66.21) (end 157 74.5) (width 0.2) (layer "F.Cu") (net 14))
 (segment (start 191 66) (end 187 66) (width 0.2) (layer "F.Cu") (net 16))
 (segment (start 191.04 65.96) (end 191 66) (width 0.2) (layer "F.Cu") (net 16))
 (segment (start 172.5 80.5) (end 172.5 93) (width 0.2) (layer "F.Cu") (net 16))
 (segment (start 187 66) (end 172.5 80.5) (width 0.2) (layer "F.Cu") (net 16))
 (segment (start 191.04 55.92) (end 191.04 65.96) (width 0.2) (layer "F.Cu") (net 16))
 (via (at 172.5 93) (size 0.6) (drill 0.3) (layers "F.Cu" "B.Cu") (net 16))
 (segment (start 159.6 102.4) (end 155.905 102.4) (width 0.2) (layer "B.Cu") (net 16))
 (segment (start 155.425 102.88) (end 155.425 103.3) (width 0.2) (layer "B.Cu") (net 16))
 (segment (start 172.5 93) (end 169 93) (width 0.2) (layer "B.Cu") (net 16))
 (segment (start 169 93) (end 159.6 102.4) (width 0.2) (layer "B.Cu") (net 16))
 (segment (start 155.905 102.4) (end 155.425 102.88) (width 0.2) (layer "B.Cu") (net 16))
 (segment (start 154.5 105.7) (end 155.285 105.7) (width 0.2) (layer "F.Cu") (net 11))
 (segment (start 151.5 102.7) (end 154.5 105.7) (width 0.2) (layer "F.Cu") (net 11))
 (segment (start 139.54 55.92) (end 151.5 67.88) (width 0.2) (layer "F.Cu") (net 11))
 (segment (start 155.285 105.7) (end 155.425 105.84) (width 0.2) (layer "F.Cu") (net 11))
 (segment (start 151.5 67.88) (end 151.5 102.7) (width 0.2) (layer "F.Cu") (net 11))
 (segment (start 170.795 116.13) (end 170.665 116) (width 0.2) (layer "F.Cu") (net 10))
 (segment (start 202.8 116.13) (end 170.795 116.13) (width 0.2) (layer "F.Cu") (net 10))
 (segment (start 209.6 101.025) (end 202.8 101.025) (width 0.2) (layer "F.Cu") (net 8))
 (segment (start 202.8 101.025) (end 202.8 105.97) (width 0.2) (layer "F.Cu") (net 8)))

